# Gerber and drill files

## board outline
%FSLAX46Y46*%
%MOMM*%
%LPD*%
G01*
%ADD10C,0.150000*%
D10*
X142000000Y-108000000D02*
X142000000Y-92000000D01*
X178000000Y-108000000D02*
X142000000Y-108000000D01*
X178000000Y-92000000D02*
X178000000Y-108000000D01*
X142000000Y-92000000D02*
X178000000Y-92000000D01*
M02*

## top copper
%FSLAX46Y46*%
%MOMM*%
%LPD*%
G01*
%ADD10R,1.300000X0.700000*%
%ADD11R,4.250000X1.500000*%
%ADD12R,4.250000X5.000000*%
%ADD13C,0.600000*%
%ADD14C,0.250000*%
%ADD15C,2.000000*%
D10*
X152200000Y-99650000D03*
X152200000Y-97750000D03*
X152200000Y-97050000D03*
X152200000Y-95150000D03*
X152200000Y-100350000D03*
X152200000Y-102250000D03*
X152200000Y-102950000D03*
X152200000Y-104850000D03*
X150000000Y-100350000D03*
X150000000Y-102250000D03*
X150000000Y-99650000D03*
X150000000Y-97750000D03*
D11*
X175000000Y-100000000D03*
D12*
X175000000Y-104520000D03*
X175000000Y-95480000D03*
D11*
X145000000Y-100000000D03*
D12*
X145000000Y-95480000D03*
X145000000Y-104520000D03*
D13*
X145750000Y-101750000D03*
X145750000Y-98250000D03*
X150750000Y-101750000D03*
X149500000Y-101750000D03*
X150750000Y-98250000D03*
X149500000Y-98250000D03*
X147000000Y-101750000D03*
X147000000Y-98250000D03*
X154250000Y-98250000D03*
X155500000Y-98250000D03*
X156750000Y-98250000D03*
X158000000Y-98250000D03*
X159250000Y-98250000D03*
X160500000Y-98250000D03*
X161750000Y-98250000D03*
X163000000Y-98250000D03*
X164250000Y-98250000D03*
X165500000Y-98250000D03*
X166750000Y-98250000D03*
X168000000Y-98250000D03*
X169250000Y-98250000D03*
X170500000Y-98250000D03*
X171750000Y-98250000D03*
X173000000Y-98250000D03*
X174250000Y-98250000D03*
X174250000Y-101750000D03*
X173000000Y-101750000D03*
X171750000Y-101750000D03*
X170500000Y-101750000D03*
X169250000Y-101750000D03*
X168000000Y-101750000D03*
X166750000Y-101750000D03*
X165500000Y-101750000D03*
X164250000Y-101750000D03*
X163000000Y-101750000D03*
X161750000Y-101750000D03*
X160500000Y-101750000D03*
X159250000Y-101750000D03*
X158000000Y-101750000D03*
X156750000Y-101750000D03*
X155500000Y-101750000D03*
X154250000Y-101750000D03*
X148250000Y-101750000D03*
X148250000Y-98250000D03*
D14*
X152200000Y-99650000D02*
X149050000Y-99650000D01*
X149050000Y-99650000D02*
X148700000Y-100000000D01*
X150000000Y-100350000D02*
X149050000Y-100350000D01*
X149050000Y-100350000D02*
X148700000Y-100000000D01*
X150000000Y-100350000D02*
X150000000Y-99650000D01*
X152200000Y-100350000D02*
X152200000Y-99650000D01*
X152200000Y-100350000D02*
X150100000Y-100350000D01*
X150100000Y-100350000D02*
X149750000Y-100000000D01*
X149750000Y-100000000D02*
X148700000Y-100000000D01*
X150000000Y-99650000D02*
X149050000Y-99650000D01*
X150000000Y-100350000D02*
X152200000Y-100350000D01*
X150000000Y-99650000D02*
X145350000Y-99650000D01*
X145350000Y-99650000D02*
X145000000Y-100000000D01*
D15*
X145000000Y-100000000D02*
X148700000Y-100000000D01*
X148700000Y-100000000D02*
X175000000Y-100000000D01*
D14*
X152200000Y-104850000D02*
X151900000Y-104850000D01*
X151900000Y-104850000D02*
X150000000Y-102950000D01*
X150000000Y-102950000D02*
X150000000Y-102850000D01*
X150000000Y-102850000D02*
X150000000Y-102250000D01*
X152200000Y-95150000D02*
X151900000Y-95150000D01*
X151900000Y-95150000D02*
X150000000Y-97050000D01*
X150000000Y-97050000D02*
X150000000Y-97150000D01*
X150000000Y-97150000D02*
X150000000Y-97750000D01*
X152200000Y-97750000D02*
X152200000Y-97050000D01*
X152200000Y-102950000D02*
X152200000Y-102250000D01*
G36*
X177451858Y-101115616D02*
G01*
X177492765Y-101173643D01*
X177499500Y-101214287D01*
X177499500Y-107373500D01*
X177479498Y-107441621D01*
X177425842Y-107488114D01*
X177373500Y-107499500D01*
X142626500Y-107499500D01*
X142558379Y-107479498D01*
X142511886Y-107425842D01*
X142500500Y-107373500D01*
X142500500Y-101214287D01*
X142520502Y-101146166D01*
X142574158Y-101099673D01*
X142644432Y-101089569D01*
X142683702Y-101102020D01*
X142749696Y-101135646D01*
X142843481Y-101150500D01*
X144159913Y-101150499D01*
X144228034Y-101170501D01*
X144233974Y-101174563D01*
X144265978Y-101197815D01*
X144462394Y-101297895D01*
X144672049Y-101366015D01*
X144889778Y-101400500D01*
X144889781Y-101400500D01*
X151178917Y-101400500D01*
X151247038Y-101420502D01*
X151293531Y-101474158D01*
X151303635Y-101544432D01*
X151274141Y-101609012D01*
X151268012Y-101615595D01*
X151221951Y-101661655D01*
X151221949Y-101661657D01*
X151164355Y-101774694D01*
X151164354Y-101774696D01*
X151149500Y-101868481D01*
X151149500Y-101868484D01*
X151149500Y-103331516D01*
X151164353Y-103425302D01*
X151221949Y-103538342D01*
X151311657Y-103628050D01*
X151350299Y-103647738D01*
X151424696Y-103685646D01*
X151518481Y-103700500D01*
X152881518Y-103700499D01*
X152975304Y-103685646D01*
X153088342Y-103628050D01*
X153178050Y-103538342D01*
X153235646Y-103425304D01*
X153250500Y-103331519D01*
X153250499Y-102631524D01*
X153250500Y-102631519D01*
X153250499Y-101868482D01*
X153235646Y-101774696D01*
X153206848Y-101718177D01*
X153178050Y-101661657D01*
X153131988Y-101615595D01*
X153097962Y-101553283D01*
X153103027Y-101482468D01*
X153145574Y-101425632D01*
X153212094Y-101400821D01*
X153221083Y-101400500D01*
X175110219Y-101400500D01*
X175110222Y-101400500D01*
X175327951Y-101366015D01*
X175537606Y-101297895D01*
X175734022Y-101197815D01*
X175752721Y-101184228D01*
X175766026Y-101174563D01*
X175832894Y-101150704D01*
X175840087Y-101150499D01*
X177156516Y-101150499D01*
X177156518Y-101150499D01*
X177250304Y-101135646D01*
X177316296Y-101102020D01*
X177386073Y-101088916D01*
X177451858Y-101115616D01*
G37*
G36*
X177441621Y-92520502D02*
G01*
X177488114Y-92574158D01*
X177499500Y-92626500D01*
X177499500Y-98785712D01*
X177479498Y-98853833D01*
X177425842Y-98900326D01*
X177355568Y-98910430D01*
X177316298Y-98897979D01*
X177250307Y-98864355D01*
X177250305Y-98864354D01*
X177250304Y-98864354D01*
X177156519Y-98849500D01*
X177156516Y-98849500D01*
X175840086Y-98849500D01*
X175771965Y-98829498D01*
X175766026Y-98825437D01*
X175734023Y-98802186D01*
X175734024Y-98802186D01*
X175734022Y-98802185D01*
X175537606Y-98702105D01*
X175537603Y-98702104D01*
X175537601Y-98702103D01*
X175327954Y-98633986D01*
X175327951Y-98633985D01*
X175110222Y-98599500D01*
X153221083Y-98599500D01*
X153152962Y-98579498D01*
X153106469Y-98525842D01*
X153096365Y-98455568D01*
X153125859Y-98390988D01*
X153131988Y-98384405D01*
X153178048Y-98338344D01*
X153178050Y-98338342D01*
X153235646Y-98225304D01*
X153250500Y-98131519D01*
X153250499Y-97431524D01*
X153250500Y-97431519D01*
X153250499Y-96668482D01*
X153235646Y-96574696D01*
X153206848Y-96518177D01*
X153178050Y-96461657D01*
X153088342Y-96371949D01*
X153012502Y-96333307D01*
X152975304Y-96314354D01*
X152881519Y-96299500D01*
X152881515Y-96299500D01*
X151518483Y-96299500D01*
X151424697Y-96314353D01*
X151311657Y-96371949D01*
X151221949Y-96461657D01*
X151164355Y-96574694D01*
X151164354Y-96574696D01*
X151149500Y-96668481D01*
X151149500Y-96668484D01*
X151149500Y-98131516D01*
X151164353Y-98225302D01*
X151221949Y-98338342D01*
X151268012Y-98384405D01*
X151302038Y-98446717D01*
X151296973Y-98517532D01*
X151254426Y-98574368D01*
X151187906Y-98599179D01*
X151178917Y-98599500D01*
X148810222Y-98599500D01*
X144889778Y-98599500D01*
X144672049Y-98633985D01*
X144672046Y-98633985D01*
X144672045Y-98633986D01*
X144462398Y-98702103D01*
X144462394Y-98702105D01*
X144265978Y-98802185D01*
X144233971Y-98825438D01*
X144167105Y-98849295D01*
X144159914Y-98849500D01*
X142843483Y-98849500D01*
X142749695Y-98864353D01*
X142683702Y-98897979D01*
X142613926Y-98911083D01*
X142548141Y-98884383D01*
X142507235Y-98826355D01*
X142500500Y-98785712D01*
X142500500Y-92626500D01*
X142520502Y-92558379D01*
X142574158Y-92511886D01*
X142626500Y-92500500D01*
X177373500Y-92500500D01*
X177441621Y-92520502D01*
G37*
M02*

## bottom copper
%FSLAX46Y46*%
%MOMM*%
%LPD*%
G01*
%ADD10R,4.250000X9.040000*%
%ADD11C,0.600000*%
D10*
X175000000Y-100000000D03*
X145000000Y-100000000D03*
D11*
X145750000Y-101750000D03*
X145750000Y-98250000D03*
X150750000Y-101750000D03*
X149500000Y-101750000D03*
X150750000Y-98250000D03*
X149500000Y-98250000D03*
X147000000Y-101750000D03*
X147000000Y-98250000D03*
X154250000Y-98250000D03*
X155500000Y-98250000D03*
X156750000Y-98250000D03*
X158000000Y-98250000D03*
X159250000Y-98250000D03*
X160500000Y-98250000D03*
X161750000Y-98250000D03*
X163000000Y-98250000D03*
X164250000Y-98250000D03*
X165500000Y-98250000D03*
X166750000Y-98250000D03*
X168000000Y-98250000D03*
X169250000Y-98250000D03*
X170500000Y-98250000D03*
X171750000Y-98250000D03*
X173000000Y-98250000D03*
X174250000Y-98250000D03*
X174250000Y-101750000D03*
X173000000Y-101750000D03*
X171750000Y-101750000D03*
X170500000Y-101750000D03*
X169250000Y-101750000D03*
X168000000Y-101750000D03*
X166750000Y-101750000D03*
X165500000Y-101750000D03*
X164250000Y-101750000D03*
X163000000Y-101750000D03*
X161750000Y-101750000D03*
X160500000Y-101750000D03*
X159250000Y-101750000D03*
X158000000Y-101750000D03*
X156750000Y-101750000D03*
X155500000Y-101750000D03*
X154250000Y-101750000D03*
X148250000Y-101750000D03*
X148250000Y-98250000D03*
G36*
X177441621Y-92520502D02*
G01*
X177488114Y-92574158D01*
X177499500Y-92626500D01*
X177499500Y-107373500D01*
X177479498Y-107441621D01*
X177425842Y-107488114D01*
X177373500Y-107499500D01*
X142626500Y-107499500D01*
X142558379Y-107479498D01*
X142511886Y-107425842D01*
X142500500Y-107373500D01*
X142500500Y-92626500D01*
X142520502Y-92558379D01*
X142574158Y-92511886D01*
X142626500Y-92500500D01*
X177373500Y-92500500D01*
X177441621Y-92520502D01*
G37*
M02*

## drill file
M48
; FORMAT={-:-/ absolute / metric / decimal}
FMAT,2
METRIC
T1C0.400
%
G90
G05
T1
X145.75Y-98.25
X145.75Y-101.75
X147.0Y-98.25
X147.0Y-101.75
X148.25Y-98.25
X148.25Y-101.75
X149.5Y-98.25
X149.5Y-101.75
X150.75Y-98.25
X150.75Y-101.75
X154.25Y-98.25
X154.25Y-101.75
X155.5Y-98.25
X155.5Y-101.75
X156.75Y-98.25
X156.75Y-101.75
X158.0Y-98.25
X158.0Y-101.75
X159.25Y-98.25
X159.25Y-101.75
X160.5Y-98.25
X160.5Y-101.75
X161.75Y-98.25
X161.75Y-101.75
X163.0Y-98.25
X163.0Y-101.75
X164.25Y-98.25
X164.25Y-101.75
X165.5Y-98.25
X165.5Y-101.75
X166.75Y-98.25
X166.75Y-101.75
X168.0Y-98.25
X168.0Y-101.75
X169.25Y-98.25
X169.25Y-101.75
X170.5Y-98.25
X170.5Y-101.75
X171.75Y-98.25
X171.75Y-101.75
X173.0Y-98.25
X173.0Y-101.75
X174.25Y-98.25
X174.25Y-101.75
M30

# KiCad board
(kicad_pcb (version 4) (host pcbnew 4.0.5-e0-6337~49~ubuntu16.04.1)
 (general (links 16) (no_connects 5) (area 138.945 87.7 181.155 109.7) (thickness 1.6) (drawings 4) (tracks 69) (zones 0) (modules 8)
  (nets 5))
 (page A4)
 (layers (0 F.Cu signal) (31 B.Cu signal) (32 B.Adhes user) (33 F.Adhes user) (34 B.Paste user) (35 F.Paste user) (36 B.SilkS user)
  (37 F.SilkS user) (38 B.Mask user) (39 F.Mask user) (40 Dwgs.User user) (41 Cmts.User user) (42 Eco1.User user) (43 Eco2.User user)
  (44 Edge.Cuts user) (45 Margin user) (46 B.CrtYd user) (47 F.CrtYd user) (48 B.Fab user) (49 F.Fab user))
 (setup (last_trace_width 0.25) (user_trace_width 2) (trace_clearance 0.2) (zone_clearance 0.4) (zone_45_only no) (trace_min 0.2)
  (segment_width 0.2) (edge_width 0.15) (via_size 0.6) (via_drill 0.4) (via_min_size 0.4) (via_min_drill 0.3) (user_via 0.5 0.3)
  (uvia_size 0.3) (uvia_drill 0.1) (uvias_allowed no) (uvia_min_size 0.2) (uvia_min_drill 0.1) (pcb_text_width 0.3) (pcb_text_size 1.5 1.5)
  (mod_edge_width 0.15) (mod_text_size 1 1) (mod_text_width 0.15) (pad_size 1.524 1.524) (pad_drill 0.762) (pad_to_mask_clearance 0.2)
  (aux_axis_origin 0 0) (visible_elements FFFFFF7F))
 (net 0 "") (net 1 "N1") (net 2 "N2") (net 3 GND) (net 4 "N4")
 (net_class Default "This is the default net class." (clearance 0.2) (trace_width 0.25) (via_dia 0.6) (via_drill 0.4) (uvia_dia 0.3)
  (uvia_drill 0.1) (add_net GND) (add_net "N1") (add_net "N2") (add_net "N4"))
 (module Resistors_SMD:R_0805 (layer F.Cu) (at 152.2 98.7 90)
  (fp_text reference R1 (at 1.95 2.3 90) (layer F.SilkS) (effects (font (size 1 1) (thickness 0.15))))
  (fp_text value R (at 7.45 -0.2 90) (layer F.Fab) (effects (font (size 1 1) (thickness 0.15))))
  (pad 1 smd rect (at -0.95 0 90) (size 0.7 1.3) (layers F.Cu F.Paste F.Mask) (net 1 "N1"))
  (pad 2 smd rect (at 0.95 0 90) (size 0.7 1.3) (layers F.Cu F.Paste F.Mask) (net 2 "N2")))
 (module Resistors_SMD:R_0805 (layer F.Cu) (at 152.2 96.1 90)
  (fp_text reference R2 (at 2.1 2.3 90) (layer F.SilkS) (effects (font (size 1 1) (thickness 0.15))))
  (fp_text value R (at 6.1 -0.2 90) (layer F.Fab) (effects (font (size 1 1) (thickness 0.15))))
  (pad 1 smd rect (at -0.95 0 90) (size 0.7 1.3) (layers F.Cu F.Paste F.Mask) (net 2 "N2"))
  (pad 2 smd rect (at 0.95 0 90) (size 0.7 1.3) (layers F.Cu F.Paste F.Mask) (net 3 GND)))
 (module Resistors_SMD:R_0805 (layer F.Cu) (at 152.2 101.3 270)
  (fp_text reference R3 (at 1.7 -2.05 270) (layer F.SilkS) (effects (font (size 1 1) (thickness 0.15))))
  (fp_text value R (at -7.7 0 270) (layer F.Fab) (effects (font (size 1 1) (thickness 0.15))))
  (pad 1 smd rect (at -0.95 0 270) (size 0.7 1.3) (layers F.Cu F.Paste F.Mask) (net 1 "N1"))
  (pad 2 smd rect (at 0.95 0 270) (size 0.7 1.3) (layers F.Cu F.Paste F.Mask) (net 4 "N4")))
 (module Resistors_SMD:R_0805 (layer F.Cu) (at 152.2 103.9 270)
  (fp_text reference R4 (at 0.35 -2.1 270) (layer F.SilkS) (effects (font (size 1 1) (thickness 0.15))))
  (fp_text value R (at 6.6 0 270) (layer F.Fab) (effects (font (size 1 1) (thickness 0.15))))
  (pad 1 smd rect (at -0.95 0 270) (size 0.7 1.3) (layers F.Cu F.Paste F.Mask) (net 4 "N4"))
  (pad 2 smd rect (at 0.95 0 270) (size 0.7 1.3) (layers F.Cu F.Paste F.Mask) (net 3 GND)))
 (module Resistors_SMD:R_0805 (layer F.Cu) (at 150 101.3 270)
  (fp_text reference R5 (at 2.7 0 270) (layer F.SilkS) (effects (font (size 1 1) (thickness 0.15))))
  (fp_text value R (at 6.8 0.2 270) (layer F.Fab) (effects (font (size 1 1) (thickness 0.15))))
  (pad 1 smd rect (at -0.95 0 270) (size 0.7 1.3) (layers F.Cu F.Paste F.Mask) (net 1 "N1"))
  (pad 2 smd rect (at 0.95 0 270) (size 0.7 1.3) (layers F.Cu F.Paste F.Mask) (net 3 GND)))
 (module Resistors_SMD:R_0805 (layer F.Cu) (at 150 98.7 90)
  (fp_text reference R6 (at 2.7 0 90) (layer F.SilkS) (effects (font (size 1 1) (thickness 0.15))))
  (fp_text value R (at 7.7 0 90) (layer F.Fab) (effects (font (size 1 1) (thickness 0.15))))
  (pad 1 smd rect (at -0.95 0 90) (size 0.7 1.3) (layers F.Cu F.Paste F.Mask) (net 1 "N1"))
  (pad 2 smd rect (at 0.95 0 90) (size 0.7 1.3) (layers F.Cu F.Paste F.Mask) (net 3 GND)))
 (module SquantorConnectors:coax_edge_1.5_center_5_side (layer F.Cu) (at 175 100 90)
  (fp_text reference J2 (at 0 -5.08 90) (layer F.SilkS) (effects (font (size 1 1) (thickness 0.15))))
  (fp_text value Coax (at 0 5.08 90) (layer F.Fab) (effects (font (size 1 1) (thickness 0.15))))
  (pad 2 smd rect (at 0 0 90) (size 1.5 4.25) (layers F.Cu F.Paste F.Mask) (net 1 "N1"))
  (pad 1 smd rect (at -4.52 0 90) (size 5 4.25) (layers F.Cu F.Paste F.Mask) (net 3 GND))
  (pad 1 smd rect (at 4.52 0 90) (size 5 4.25) (layers F.Cu F.Paste F.Mask) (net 3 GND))
  (pad 1 smd rect (at 0 0 90) (size 9.04 4.25) (layers B.Cu B.Paste B.Mask) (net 3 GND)))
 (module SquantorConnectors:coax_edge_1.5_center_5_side (layer F.Cu) (at 145 100 270)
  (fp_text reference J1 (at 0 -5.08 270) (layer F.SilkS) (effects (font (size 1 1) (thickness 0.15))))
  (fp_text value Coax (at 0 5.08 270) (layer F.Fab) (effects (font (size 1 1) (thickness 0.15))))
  (pad 2 smd rect (at 0 0 270) (size 1.5 4.25) (layers F.Cu F.Paste F.Mask) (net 1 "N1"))
  (pad 1 smd rect (at -4.52 0 270) (size 5 4.25) (layers F.Cu F.Paste F.Mask) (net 3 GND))
  (pad 1 smd rect (at 4.52 0 270) (size 5 4.25) (layers F.Cu F.Paste F.Mask) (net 3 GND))
  (pad 1 smd rect (at 0 0 270) (size 9.04 4.25) (layers B.Cu B.Paste B.Mask) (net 3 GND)))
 (gr_line (start 142 108) (end 142 92) (layer Edge.Cuts) (width 0.15))
 (gr_line (start 178 108) (end 142 108) (layer Edge.Cuts) (width 0.15))
 (gr_line (start 178 92) (end 178 108) (layer Edge.Cuts) (width 0.15))
 (gr_line (start 142 92) (end 178 92) (layer Edge.Cuts) (width 0.15))
 (segment (start 152.2 99.65) (end 149.05 99.65) (width 0.25) (layer F.Cu) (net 1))
 (segment (start 149.05 99.65) (end 148.7 100) (width 0.25) (layer F.Cu) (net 1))
 (segment (start 150 100.35) (end 149.05 100.35) (width 0.25) (layer F.Cu) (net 1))
 (segment (start 149.05 100.35) (end 148.7 100) (width 0.25) (layer F.Cu) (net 1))
 (segment (start 150 100.35) (end 150 99.65) (width 0.25) (layer F.Cu) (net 1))
 (segment (start 152.2 100.35) (end 152.2 99.65) (width 0.25) (layer F.Cu) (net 1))
 (segment (start 152.2 100.35) (end 150.1 100.35) (width 0.25) (layer F.Cu) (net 1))
 (segment (start 150.1 100.35) (end 149.75 100) (width 0.25) (layer F.Cu) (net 1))
 (segment (start 149.75 100) (end 148.7 100) (width 0.25) (layer F.Cu) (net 1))
 (segment (start 150 99.65) (end 149.05 99.65) (width 0.25) (layer F.Cu) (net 1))
 (segment (start 150 100.35) (end 152.2 100.35) (width 0.25) (layer F.Cu) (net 1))
 (segment (start 150 99.65) (end 145.35 99.65) (width 0.25) (layer F.Cu) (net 1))
 (segment (start 145.35 99.65) (end 145 100) (width 0.25) (layer F.Cu) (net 1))
 (segment (start 145 100) (end 148.7 100) (width 2) (layer F.Cu) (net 1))
 (segment (start 148.7 100) (end 175 100) (width 2) (layer F.Cu) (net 1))
 (via (at 145.75 101.75) (size 0.6) (drill 0.4) (layers F.Cu B.Cu) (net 3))
 (via (at 145.75 98.25) (size 0.6) (drill 0.4) (layers F.Cu B.Cu) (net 3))
 (via (at 150.75 101.75) (size 0.6) (drill 0.4) (layers F.Cu B.Cu) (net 3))
 (via (at 149.5 101.75) (size 0.6) (drill 0.4) (layers F.Cu B.Cu) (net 3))
 (via (at 150.75 98.25) (size 0.6) (drill 0.4) (layers F.Cu B.Cu) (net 3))
 (via (at 149.5 98.25) (size 0.6) (drill 0.4) (layers F.Cu B.Cu) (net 3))
 (via (at 147 101.75) (size 0.6) (drill 0.4) (layers F.Cu B.Cu) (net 3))
 (via (at 147 98.25) (size 0.6) (drill 0.4) (layers F.Cu B.Cu) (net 3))
 (via (at 154.25 98.25) (size 0.6) (drill 0.4) (layers F.Cu B.Cu) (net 3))
 (via (at 155.5 98.25) (size 0.6) (drill 0.4) (layers F.Cu B.Cu) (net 3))
 (via (at 156.75 98.25) (size 0.6) (drill 0.4) (layers F.Cu B.Cu) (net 3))
 (via (at 158 98.25) (size 0.6) (drill 0.4) (layers F.Cu B.Cu) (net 3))
 (via (at 159.25 98.25) (size 0.6) (drill 0.4) (layers F.Cu B.Cu) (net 3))
 (via (at 160.5 98.25) (size 0.6) (drill 0.4) (layers F.Cu B.Cu) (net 3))
 (via (at 161.75 98.25) (size 0.6) (drill 0.4) (layers F.Cu B.Cu) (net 3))
 (via (at 163 98.25) (size 0.6) (drill 0.4) (layers F.Cu B.Cu) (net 3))
 (via (at 164.25 98.25) (size 0.6) (drill 0.4) (layers F.Cu B.Cu) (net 3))
 (via (at 165.5 98.25) (size 0.6) (drill 0.4) (layers F.Cu B.Cu) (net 3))
 (via (at 166.75 98.25) (size 0.6) (drill 0.4) (layers F.Cu B.Cu) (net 3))
 (via (at 168 98.25) (size 0.6) (drill 0.4) (layers F.Cu B.Cu) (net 3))
 (via (at 169.25 98.25) (size 0.6) (drill 0.4) (layers F.Cu B.Cu) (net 3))
 (via (at 170.5 98.25) (size 0.6) (drill 0.4) (layers F.Cu B.Cu) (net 3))
 (via (at 171.75 98.25) (size 0.6) (drill 0.4) (layers F.Cu B.Cu) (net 3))
 (via (at 173 98.25) (size 0.6) (drill 0.4) (layers F.Cu B.Cu) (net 3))
 (via (at 174.25 98.25) (size 0.6) (drill 0.4) (layers F.Cu B.Cu) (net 3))
 (via (at 174.25 101.75) (size 0.6) (drill 0.4) (layers F.Cu B.Cu) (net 3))
 (via (at 173 101.75) (size 0.6) (drill 0.4) (layers F.Cu B.Cu) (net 3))
 (via (at 171.75 101.75) (size 0.6) (drill 0.4) (layers F.Cu B.Cu) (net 3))
 (via (at 170.5 101.75) (size 0.6) (drill 0.4) (layers F.Cu B.Cu) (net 3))
 (via (at 169.25 101.75) (size 0.6) (drill 0.4) (layers F.Cu B.Cu) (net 3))
 (via (at 168 101.75) (size 0.6) (drill 0.4) (layers F.Cu B.Cu) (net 3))
 (via (at 166.75 101.75) (size 0.6) (drill 0.4) (layers F.Cu B.Cu) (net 3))
 (via (at 165.5 101.75) (size 0.6) (drill 0.4) (layers F.Cu B.Cu) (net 3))
 (via (at 164.25 101.75) (size 0.6) (drill 0.4) (layers F.Cu B.Cu) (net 3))
 (via (at 163 101.75) (size 0.6) (drill 0.4) (layers F.Cu B.Cu) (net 3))
 (via (at 161.75 101.75) (size 0.6) (drill 0.4) (layers F.Cu B.Cu) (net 3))
 (via (at 160.5 101.75) (size 0.6) (drill 0.4) (layers F.Cu B.Cu) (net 3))
 (via (at 159.25 101.75) (size 0.6) (drill 0.4) (layers F.Cu B.Cu) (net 3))
 (via (at 158 101.75) (size 0.6) (drill 0.4) (layers F.Cu B.Cu) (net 3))
 (via (at 156.75 101.75) (size 0.6) (drill 0.4) (layers F.Cu B.Cu) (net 3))
 (via (at 155.5 101.75) (size 0.6) (drill 0.4) (layers F.Cu B.Cu) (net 3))
 (via (at 154.25 101.75) (size 0.6) (drill 0.4) (layers F.Cu B.Cu) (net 3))
 (via (at 148.25 101.75) (size 0.6) (drill 0.4) (layers F.Cu B.Cu) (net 3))
 (via (at 148.25 98.25) (size 0.6) (drill 0.4) (layers F.Cu B.Cu) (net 3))
 (segment (start 152.2 104.85) (end 151.9 104.85) (width 0.25) (layer F.Cu) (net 3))
 (segment (start 151.9 104.85) (end 150 102.95) (width 0.25) (layer F.Cu) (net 3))
 (segment (start 150 102.95) (end 150 102.85) (width 0.25) (layer F.Cu) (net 3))
 (segment (start 150 102.85) (end 150 102.25) (width 0.25) (layer F.Cu) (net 3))
 (segment (start 152.2 95.15) (end 151.9 95.15) (width 0.25) (layer F.Cu) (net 3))
 (segment (start 151.9 95.15) (end 150 97.05) (width 0.25) (layer F.Cu) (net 3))
 (segment (start 150 97.05) (end 150 97.15) (width 0.25) (layer F.Cu) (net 3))
 (segment (start 150 97.15) (end 150 97.75) (width 0.25) (layer F.Cu) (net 3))
 (segment (start 152.2 97.75) (end 152.2 97.05) (width 0.25) (layer F.Cu) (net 2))
 (segment (start 152.2 102.95) (end 152.2 102.25) (width 0.25) (layer F.Cu) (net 4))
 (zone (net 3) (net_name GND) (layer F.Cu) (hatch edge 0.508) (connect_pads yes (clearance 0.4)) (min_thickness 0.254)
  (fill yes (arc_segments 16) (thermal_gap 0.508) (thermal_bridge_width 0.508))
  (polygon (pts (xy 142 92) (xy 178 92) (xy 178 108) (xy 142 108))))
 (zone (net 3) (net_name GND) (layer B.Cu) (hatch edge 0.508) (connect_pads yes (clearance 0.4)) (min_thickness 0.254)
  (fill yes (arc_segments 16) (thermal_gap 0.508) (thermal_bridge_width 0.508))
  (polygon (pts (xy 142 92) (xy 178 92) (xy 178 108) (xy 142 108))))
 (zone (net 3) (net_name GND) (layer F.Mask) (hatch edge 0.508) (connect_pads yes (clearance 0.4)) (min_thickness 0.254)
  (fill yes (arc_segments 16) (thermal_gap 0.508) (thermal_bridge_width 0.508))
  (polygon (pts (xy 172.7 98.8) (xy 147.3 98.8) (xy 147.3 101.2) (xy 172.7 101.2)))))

